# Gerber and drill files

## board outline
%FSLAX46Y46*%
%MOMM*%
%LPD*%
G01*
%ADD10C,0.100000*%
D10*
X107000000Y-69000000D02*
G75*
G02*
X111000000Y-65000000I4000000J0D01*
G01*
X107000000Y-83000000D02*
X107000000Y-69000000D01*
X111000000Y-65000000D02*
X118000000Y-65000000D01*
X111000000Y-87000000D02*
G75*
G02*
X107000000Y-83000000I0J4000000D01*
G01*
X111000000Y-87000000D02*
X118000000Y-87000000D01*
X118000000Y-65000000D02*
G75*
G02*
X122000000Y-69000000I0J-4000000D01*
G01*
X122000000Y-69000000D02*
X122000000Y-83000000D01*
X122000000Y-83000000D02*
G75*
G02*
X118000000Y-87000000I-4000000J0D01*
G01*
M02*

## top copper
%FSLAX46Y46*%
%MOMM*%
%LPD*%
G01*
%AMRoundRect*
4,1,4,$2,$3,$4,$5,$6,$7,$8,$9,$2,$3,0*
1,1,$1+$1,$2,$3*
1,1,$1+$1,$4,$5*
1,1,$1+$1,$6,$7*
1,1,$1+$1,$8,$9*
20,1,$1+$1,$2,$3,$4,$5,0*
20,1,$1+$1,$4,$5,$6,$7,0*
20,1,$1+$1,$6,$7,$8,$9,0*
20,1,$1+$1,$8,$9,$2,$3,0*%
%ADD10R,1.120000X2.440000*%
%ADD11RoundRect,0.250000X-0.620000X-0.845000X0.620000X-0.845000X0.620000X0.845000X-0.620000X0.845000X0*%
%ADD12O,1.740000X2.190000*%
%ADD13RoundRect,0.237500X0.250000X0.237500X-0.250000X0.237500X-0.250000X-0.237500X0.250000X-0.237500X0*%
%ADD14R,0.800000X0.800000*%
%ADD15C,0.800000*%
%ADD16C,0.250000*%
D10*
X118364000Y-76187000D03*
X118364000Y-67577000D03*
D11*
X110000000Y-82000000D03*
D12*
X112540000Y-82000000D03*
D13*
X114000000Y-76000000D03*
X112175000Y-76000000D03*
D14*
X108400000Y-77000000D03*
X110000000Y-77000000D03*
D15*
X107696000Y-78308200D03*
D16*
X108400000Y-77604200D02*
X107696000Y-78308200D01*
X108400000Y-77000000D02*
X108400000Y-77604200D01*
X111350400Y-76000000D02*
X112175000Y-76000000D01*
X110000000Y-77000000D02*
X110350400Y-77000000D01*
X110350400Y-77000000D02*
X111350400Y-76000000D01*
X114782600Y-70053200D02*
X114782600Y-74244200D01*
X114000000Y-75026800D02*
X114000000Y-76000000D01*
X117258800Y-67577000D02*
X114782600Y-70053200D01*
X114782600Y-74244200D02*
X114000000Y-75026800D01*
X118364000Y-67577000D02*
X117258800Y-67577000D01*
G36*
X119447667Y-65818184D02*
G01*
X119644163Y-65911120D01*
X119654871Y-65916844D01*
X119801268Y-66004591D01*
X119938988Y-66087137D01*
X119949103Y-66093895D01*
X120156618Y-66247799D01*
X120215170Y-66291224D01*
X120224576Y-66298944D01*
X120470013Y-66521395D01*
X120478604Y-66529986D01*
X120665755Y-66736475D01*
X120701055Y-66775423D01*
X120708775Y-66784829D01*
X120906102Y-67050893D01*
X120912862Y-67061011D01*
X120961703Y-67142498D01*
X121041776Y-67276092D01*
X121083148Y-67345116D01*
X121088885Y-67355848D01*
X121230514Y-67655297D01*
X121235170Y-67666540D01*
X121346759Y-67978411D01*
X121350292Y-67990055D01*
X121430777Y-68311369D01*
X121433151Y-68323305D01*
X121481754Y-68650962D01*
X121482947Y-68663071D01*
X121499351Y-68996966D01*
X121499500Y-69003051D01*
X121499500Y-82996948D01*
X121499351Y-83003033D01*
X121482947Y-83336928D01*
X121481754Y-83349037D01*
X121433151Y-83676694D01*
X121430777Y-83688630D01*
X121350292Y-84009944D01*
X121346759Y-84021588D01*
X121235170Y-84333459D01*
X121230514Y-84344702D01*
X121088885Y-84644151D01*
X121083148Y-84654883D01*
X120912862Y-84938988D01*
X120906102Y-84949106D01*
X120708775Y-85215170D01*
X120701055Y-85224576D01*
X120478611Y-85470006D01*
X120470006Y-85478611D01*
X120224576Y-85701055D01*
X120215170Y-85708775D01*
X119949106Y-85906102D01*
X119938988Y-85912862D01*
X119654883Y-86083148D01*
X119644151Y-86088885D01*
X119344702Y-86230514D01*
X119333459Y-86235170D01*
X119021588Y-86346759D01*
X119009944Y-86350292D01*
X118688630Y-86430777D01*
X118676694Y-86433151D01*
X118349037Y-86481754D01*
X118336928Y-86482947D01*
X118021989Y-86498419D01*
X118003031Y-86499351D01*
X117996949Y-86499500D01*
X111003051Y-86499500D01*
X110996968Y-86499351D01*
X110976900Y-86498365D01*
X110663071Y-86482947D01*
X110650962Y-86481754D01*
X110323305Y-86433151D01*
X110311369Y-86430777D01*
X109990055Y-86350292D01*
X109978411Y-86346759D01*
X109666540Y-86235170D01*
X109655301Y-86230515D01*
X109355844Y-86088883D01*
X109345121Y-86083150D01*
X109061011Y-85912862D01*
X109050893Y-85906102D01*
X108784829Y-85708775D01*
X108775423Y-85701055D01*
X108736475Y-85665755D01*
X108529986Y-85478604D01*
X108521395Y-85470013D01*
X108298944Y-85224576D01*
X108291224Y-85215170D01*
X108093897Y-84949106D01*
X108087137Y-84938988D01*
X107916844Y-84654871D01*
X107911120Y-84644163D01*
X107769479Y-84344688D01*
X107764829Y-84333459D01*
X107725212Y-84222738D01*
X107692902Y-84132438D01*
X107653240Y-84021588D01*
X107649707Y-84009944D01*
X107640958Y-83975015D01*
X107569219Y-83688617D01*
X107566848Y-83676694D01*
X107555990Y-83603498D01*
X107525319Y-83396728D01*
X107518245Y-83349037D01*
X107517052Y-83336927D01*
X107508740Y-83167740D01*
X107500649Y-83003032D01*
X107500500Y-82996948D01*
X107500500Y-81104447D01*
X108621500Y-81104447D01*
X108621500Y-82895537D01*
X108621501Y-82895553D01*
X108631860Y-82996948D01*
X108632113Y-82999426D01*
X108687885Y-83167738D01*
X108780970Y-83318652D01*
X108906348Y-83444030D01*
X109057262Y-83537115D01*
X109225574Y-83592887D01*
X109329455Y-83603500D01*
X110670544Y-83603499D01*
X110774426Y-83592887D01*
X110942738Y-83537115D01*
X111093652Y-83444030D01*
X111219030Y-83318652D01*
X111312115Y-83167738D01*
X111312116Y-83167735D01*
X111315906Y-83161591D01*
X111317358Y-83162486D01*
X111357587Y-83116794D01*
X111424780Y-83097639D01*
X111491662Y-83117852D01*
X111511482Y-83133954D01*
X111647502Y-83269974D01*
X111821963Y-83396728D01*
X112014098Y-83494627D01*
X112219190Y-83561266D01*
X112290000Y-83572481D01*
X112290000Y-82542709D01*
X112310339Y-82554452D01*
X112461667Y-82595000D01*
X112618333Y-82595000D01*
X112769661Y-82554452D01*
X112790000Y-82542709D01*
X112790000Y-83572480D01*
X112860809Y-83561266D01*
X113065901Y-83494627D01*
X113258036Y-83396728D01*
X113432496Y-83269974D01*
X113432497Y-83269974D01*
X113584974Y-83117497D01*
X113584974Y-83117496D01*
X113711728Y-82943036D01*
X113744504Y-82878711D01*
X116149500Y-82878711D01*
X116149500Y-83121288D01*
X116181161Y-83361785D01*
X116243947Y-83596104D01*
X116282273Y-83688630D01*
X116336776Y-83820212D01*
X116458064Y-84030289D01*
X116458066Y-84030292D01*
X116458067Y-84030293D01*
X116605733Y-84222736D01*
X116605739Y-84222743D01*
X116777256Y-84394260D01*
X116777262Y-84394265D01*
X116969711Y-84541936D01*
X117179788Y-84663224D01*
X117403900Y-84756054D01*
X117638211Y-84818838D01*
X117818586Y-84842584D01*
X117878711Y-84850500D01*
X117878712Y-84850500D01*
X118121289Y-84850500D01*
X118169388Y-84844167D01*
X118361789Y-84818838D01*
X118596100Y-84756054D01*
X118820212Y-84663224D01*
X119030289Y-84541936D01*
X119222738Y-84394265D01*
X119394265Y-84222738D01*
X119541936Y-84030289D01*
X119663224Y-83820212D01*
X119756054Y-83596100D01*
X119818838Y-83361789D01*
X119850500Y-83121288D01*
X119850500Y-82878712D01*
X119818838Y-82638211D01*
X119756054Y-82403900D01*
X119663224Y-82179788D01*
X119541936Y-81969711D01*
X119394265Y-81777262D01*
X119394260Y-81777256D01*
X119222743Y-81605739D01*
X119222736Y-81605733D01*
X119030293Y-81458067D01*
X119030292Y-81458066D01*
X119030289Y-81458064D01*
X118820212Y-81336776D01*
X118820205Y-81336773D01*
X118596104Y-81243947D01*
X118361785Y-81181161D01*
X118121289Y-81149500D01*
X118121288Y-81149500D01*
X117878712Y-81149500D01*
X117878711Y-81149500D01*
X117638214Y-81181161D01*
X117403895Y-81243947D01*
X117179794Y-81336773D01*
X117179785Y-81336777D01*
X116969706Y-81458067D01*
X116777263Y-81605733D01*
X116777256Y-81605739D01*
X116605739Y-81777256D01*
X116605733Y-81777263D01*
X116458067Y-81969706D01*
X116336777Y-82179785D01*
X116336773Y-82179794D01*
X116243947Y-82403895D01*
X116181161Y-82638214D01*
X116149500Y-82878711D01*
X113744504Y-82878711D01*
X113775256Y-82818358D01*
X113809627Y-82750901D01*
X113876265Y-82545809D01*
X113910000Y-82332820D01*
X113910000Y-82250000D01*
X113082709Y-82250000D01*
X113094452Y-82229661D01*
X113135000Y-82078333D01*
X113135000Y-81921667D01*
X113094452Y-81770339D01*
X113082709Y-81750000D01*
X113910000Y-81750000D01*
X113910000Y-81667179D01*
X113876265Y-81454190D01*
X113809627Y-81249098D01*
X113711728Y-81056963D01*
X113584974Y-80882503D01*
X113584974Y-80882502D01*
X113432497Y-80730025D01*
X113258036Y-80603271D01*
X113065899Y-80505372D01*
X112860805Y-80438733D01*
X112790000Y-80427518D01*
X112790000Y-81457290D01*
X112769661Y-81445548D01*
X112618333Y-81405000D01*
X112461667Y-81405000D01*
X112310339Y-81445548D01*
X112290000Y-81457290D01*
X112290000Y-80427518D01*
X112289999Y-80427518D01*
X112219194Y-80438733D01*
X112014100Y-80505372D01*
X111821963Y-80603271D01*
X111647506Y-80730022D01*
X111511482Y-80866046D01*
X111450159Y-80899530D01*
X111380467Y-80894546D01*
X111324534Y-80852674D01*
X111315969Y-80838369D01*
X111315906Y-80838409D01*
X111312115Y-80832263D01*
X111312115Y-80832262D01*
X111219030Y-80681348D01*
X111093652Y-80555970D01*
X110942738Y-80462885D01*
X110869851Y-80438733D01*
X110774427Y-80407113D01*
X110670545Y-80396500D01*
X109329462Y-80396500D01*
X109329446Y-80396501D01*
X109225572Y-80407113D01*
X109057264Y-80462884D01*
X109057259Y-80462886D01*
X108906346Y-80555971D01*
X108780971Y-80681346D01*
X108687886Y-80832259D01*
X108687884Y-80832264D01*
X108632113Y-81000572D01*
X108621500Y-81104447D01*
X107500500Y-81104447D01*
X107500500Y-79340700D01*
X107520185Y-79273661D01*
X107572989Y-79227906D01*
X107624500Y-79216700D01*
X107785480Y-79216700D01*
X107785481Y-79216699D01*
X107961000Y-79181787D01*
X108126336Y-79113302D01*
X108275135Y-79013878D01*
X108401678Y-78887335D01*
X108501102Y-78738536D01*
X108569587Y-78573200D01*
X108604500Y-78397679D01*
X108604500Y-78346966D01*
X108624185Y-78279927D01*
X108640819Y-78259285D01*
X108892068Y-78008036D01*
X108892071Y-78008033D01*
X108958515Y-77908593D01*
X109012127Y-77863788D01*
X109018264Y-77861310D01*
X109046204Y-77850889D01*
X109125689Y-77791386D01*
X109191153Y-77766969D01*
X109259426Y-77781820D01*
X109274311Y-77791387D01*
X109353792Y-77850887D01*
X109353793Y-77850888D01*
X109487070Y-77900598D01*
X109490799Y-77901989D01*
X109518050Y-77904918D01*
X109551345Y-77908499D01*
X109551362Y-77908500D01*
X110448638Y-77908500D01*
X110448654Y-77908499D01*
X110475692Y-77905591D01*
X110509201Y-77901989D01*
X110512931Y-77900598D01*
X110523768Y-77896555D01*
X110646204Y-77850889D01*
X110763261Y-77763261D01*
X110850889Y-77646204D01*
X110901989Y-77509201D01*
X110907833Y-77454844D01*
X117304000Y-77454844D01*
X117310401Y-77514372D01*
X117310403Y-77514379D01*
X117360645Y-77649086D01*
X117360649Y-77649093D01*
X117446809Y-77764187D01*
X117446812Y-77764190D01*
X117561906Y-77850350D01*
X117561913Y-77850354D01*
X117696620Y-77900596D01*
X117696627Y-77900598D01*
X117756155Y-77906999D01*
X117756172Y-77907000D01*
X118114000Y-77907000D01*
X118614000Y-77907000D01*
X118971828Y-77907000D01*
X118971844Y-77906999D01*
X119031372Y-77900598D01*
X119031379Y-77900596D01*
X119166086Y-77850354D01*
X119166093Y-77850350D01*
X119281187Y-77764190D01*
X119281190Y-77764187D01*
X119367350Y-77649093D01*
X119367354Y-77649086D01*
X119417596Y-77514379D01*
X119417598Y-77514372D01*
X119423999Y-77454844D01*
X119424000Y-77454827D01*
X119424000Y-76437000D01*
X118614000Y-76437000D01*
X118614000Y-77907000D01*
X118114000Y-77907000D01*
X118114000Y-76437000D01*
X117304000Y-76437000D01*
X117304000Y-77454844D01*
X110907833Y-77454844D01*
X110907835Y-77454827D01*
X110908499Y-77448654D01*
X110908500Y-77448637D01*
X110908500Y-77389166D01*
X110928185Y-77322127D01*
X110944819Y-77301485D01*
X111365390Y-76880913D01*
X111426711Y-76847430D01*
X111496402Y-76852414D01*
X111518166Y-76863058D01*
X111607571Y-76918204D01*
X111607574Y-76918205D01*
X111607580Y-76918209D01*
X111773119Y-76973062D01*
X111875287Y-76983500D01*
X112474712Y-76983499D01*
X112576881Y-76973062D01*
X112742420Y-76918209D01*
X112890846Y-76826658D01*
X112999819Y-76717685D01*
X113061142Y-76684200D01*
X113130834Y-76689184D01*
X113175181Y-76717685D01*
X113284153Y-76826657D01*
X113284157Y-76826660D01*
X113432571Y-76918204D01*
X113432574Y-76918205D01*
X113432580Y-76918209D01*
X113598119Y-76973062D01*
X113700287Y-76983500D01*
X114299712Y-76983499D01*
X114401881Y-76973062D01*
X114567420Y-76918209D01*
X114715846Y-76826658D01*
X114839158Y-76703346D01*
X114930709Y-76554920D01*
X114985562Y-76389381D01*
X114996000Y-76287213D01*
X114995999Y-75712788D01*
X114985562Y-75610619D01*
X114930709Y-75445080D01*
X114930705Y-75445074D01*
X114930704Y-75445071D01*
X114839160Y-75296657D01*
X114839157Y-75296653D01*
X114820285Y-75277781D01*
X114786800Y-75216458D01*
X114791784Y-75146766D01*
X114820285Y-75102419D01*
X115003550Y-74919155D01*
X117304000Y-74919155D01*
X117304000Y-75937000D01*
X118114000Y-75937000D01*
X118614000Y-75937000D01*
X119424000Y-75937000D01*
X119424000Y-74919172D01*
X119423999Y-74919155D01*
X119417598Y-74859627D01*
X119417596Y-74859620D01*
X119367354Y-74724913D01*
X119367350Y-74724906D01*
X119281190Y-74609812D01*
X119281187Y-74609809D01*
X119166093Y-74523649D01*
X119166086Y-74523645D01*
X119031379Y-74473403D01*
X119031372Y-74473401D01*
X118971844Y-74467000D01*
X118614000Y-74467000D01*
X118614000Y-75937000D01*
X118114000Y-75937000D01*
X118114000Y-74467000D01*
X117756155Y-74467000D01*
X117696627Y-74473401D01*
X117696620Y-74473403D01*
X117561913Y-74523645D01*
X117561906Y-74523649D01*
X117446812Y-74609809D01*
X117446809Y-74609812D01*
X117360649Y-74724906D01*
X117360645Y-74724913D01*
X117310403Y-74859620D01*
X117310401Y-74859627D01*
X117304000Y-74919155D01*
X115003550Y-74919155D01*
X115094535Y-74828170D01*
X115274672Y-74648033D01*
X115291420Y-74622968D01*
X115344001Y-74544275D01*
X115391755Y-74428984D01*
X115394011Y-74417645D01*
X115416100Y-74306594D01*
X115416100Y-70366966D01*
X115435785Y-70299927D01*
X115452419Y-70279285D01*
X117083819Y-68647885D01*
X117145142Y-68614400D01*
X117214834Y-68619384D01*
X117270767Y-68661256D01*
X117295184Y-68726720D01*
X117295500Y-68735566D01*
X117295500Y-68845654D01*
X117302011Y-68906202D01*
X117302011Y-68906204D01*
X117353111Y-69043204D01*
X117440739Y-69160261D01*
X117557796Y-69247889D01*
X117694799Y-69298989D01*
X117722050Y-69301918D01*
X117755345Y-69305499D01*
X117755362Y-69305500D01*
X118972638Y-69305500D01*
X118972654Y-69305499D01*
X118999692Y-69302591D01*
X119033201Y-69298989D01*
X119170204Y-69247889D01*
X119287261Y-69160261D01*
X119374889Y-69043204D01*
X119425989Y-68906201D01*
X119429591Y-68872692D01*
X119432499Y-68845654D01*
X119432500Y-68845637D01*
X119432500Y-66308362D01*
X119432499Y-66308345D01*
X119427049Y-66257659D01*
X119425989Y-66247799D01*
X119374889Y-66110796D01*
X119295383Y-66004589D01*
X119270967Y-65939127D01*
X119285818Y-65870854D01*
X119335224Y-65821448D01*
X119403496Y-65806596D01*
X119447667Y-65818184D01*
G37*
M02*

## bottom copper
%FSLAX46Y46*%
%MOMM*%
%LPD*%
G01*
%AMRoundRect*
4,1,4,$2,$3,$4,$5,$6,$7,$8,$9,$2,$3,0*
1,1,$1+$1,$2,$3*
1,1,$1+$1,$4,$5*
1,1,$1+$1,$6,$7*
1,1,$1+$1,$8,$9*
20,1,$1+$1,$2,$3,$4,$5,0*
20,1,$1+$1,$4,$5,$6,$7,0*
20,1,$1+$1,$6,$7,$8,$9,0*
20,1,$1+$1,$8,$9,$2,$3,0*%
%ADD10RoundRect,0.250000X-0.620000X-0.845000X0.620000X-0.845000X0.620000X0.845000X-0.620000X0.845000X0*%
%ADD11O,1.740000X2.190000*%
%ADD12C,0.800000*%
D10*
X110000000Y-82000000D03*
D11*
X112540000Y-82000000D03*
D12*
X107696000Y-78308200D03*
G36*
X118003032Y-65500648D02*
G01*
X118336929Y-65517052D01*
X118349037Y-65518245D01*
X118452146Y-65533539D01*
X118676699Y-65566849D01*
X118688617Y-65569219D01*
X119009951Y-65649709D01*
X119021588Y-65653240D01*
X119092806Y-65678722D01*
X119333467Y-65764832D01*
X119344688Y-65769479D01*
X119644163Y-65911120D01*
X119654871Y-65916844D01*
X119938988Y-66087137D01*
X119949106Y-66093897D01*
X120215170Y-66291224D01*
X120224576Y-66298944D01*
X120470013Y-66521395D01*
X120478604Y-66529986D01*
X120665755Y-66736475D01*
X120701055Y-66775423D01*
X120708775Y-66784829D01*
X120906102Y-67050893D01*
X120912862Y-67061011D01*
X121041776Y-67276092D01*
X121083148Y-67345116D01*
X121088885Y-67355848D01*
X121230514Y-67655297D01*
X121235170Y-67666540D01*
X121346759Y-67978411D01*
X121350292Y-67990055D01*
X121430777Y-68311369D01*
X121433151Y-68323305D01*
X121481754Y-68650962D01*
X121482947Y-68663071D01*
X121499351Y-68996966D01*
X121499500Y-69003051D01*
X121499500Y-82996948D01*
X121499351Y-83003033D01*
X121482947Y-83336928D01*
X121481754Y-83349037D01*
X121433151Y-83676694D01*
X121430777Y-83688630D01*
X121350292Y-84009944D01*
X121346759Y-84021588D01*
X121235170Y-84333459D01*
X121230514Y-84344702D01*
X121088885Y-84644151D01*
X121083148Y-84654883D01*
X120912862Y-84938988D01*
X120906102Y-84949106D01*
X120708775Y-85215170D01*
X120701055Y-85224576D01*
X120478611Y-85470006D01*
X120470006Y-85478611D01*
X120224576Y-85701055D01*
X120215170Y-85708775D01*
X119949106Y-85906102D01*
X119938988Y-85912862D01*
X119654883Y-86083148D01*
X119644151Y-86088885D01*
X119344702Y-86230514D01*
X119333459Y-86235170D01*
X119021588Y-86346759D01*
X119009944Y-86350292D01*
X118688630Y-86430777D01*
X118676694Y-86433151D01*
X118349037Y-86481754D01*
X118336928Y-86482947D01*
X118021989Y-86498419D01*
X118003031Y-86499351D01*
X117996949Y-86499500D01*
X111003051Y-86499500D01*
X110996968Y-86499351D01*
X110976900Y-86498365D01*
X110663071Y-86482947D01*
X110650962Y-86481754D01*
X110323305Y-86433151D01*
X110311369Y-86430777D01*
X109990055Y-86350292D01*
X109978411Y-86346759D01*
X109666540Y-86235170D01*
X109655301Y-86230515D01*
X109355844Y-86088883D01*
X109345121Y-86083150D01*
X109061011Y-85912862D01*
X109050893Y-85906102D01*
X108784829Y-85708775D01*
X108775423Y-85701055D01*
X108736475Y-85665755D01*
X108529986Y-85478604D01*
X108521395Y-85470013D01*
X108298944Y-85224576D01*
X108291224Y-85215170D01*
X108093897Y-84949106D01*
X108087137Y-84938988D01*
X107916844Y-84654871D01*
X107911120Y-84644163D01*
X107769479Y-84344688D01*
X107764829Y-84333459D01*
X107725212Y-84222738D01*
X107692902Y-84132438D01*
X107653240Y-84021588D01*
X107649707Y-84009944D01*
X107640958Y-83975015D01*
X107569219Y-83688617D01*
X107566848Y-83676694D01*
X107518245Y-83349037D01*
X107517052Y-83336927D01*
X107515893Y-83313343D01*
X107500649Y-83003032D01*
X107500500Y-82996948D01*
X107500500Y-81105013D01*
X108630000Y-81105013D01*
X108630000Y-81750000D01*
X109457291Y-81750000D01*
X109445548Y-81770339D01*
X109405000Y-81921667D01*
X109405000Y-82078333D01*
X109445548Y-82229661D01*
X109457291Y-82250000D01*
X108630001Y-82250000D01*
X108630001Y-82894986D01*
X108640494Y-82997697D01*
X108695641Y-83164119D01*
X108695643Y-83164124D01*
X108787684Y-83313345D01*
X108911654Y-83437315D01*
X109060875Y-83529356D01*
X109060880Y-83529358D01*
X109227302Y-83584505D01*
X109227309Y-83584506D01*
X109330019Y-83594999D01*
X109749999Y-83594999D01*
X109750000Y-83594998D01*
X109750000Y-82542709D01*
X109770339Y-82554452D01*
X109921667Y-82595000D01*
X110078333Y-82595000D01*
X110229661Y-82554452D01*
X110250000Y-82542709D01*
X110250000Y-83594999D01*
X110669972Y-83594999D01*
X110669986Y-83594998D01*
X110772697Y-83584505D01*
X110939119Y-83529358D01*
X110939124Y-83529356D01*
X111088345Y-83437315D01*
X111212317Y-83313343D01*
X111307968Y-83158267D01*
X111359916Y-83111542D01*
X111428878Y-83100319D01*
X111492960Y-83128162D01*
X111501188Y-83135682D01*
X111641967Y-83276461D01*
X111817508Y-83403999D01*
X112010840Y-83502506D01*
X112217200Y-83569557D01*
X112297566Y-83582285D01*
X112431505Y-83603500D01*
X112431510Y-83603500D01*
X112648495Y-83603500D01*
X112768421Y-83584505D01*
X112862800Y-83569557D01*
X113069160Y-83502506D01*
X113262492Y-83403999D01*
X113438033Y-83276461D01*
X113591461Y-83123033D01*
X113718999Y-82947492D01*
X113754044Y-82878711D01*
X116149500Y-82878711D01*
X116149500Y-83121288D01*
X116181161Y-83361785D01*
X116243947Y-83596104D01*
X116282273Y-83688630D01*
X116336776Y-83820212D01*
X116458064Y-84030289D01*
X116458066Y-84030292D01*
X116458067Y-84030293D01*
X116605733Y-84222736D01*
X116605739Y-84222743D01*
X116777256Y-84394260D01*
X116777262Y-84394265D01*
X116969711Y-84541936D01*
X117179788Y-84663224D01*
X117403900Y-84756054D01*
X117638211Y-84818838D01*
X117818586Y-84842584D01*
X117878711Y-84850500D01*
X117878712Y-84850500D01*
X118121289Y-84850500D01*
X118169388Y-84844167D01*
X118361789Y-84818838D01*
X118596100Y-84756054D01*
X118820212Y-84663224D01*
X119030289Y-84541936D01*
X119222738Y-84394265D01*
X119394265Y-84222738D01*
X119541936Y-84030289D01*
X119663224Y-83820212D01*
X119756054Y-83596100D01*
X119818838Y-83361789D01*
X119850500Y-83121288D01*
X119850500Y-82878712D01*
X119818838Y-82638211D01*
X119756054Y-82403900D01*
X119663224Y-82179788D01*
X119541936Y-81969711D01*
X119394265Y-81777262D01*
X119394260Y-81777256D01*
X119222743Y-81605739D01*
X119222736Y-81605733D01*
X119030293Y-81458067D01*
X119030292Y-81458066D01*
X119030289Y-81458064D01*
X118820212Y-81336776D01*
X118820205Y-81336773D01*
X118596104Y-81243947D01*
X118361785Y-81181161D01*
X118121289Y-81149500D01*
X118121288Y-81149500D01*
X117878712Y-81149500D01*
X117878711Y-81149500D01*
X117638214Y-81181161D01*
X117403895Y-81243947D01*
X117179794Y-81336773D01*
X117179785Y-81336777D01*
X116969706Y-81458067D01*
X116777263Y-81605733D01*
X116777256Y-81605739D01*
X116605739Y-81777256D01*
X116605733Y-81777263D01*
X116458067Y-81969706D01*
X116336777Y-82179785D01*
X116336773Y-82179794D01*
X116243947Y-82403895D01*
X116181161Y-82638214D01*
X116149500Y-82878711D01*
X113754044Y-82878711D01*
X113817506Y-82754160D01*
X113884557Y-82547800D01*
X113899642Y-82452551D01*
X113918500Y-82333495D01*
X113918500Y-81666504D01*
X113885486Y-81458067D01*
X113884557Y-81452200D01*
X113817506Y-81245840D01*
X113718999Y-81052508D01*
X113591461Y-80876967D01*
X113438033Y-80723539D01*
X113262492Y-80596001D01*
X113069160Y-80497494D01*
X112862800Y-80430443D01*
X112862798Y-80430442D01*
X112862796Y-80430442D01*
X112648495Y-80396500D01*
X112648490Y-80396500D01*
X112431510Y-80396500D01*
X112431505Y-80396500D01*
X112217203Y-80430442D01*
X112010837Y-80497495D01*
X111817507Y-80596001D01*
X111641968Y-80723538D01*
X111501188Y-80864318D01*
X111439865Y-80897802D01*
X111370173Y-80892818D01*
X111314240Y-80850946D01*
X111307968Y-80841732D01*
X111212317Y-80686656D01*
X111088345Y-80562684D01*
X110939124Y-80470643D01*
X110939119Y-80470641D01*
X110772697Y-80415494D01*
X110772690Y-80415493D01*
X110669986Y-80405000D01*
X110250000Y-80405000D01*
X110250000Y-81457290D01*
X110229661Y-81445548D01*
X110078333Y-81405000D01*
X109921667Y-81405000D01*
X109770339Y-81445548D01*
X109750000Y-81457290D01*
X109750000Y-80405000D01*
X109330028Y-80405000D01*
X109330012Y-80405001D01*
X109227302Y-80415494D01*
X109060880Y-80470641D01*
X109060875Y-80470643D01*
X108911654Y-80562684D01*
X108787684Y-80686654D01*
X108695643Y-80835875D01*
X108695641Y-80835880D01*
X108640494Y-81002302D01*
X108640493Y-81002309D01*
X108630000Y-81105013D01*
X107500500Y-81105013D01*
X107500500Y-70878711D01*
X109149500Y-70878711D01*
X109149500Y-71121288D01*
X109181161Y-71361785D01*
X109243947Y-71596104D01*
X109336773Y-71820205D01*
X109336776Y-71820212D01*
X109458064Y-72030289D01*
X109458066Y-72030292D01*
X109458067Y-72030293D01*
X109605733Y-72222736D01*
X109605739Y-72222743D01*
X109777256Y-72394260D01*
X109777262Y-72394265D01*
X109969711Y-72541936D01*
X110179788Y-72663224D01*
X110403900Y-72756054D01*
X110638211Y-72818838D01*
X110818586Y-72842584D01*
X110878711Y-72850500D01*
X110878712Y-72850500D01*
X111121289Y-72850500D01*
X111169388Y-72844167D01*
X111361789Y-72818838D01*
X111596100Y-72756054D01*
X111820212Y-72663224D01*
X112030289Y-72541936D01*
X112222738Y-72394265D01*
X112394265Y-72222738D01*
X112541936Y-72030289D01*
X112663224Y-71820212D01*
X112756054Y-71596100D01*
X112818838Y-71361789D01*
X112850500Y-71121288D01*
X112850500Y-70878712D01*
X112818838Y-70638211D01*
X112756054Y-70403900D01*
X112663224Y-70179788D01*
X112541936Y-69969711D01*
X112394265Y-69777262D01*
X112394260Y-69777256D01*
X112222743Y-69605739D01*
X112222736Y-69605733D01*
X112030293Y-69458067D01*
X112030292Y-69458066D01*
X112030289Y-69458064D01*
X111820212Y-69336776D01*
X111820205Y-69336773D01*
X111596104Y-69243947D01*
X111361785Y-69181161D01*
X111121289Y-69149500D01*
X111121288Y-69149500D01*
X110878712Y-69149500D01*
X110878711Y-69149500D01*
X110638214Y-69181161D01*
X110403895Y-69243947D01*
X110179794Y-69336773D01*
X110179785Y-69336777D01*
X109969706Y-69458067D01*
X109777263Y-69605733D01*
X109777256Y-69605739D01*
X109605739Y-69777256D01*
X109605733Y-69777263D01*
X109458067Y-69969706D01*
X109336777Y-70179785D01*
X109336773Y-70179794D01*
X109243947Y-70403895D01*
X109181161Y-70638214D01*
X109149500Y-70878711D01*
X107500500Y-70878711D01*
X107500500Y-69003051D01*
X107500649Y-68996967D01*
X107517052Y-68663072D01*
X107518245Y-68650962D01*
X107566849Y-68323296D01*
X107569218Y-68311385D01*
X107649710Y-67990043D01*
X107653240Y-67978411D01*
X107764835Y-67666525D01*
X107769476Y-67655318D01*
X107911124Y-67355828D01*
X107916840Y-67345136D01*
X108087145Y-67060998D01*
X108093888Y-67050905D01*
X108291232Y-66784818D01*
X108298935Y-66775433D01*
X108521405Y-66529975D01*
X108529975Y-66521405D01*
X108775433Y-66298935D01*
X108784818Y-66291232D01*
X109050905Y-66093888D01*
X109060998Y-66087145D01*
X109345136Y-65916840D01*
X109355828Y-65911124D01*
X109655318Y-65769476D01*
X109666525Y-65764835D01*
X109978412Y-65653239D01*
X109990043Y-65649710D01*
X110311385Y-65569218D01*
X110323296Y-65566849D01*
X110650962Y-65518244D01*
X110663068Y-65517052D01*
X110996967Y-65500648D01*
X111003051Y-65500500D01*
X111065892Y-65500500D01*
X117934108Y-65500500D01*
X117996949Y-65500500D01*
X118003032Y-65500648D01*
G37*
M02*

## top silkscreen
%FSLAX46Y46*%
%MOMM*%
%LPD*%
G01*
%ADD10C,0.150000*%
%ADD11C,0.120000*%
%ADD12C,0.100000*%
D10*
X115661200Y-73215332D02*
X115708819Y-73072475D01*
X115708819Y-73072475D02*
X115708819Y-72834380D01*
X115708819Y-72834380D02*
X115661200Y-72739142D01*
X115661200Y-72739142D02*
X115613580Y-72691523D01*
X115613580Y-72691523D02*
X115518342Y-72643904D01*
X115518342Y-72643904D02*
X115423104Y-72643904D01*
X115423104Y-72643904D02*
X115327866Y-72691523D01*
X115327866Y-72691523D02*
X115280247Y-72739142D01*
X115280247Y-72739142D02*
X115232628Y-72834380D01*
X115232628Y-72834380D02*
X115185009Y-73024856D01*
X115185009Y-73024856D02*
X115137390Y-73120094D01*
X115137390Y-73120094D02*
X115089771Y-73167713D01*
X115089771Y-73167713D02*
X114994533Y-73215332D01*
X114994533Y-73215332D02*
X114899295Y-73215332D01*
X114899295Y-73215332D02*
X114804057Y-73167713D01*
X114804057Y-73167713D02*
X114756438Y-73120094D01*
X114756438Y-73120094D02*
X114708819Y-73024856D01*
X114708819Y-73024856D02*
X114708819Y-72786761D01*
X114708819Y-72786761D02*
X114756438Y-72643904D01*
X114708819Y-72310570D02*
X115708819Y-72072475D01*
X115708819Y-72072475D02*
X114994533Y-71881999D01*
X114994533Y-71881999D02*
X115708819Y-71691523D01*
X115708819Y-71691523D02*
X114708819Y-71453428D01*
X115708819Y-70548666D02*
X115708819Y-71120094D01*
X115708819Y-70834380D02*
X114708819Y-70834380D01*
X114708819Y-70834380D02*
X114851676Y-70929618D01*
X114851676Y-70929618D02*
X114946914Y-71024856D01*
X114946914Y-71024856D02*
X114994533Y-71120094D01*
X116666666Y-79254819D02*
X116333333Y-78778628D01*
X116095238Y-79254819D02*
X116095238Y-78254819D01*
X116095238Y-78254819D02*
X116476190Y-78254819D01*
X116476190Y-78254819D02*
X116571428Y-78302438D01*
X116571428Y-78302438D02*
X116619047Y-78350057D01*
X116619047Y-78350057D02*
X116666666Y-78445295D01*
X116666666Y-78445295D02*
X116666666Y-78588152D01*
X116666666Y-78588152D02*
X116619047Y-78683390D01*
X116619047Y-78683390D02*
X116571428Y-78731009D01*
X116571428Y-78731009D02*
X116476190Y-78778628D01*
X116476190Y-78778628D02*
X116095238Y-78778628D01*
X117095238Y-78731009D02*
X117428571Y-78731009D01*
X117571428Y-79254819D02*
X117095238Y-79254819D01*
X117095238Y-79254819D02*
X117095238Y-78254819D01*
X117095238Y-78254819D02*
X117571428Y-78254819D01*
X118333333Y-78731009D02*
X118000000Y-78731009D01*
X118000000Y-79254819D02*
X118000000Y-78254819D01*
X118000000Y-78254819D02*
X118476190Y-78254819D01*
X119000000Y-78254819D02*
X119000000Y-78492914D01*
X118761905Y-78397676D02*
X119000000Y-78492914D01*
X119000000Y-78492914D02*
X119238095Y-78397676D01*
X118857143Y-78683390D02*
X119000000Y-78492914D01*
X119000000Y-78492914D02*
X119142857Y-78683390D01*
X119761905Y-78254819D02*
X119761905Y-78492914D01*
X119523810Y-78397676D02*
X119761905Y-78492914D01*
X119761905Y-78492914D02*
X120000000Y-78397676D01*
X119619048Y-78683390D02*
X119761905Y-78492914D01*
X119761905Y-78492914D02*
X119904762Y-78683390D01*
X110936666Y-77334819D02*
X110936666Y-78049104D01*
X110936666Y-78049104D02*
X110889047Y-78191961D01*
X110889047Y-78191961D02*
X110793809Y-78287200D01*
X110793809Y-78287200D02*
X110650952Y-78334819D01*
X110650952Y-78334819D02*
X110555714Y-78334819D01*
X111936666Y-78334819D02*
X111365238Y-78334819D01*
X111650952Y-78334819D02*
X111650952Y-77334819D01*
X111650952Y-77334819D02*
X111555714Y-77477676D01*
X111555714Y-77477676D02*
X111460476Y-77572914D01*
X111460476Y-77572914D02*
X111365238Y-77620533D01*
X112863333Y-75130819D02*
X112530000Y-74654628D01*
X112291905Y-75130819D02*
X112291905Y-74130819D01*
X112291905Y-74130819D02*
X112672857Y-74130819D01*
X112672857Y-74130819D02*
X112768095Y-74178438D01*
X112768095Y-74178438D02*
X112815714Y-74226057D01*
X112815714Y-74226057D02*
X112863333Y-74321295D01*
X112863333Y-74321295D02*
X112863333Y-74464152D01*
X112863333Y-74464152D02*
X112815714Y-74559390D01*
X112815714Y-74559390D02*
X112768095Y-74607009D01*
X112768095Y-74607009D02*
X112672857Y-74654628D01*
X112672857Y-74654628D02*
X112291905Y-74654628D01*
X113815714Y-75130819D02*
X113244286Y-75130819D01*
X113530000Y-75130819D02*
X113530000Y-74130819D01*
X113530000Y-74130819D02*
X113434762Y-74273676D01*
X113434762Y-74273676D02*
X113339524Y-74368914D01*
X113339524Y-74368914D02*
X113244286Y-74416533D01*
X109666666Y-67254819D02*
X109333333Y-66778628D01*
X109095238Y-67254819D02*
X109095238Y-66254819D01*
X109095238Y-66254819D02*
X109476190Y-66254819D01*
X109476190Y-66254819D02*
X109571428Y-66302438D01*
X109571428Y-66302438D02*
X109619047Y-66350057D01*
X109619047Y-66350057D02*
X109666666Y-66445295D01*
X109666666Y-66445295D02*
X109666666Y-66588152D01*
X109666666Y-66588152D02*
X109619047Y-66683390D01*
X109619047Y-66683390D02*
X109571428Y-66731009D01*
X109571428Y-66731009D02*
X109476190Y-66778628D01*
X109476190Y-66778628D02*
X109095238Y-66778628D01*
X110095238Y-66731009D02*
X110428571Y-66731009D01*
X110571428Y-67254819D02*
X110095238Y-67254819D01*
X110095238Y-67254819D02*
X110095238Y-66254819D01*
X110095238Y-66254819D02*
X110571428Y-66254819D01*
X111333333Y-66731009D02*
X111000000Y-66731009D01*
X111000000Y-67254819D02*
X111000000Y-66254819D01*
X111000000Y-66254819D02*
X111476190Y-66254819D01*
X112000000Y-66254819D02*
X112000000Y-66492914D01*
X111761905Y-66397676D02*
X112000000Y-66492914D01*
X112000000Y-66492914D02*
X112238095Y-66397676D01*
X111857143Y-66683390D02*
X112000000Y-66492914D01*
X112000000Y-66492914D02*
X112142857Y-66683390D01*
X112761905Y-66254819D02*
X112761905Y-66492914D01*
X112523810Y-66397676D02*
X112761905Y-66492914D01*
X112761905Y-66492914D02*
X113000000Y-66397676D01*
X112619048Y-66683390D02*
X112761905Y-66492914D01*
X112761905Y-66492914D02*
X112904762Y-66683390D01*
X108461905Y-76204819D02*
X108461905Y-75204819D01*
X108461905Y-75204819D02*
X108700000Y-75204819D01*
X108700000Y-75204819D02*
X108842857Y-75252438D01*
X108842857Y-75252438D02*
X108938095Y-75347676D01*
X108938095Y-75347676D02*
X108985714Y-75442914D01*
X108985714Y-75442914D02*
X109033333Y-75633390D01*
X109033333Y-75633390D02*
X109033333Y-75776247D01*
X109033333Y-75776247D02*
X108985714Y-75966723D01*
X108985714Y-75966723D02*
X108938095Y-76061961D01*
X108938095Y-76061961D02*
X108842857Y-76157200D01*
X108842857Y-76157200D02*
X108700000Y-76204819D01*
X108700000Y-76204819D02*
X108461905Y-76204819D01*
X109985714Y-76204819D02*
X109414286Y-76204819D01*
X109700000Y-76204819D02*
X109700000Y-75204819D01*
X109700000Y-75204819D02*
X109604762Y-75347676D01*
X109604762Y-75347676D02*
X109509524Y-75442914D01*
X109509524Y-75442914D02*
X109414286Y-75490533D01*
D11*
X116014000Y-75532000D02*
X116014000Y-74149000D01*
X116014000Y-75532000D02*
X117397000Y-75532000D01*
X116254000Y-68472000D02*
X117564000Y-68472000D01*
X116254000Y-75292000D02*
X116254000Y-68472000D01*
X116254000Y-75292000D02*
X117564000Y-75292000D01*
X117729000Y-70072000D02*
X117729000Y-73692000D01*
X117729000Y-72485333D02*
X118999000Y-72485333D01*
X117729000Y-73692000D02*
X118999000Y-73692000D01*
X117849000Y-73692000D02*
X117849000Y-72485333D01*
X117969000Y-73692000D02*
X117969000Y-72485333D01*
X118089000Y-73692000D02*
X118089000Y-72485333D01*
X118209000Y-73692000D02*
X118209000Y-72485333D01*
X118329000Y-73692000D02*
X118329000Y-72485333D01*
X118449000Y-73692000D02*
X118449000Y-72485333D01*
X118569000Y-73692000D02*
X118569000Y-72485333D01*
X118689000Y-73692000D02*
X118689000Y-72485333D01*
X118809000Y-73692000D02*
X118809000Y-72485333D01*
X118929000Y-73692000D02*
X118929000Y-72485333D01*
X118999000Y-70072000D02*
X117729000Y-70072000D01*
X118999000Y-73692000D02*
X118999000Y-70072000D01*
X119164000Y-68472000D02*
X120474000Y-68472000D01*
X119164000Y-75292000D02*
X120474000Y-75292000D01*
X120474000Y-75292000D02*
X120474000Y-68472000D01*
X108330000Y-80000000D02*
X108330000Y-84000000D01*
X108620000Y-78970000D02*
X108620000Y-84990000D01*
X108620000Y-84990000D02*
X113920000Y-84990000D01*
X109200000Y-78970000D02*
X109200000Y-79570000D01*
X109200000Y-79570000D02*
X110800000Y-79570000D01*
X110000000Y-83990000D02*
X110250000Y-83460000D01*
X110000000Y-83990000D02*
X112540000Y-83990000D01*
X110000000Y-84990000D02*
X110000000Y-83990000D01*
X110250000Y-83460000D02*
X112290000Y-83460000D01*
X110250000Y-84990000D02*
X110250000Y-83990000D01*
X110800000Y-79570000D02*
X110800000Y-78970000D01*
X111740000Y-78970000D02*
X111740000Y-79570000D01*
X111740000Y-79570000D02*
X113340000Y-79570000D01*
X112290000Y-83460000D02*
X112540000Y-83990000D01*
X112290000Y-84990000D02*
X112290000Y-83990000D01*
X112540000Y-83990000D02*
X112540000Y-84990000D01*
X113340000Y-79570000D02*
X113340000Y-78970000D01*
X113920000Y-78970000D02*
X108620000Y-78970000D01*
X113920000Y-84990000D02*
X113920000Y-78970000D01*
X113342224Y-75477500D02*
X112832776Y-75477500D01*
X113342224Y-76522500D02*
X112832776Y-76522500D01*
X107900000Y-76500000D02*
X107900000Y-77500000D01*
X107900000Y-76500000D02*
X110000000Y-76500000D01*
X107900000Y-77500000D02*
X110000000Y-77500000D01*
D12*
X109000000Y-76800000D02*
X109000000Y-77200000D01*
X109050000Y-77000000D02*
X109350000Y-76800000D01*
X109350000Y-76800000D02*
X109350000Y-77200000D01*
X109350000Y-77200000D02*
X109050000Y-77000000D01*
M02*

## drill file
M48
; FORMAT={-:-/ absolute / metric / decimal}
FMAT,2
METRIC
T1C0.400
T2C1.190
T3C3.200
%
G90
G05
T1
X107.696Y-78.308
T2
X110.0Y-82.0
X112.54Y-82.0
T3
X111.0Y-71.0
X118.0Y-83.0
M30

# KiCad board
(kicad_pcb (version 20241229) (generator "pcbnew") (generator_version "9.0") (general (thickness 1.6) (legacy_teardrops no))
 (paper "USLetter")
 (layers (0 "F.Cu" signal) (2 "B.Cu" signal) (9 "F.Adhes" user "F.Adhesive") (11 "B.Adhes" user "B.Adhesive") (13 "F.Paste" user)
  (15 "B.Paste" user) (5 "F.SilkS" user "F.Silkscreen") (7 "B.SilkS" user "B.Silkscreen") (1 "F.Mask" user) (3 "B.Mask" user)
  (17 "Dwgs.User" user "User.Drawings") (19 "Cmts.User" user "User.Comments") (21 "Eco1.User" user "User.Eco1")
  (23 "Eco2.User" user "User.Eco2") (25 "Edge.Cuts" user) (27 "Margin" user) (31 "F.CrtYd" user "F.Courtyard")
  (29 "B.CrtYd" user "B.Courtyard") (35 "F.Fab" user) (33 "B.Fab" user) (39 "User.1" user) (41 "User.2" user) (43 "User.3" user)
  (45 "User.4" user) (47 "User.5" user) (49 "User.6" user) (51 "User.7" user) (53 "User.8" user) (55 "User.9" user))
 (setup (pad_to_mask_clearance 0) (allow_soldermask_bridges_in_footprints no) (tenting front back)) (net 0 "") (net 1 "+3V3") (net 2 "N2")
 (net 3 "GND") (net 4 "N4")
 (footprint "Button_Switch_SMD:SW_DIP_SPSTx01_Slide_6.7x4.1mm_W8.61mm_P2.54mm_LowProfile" (layer "F.Cu") (at 118.364 71.882 90)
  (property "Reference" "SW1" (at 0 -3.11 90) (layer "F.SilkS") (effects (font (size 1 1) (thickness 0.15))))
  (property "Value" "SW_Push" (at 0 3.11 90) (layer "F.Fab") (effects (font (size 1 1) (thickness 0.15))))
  (fp_line (start -3.65 -2.35) (end -2.267 -2.35) (stroke (width 0.12) (type solid)) (layer "F.SilkS"))
  (fp_line (start -3.65 -2.35) (end -3.65 -0.967) (stroke (width 0.12) (type solid)) (layer "F.SilkS"))
  (fp_line (start 3.41 -2.11) (end 3.41 -0.8) (stroke (width 0.12) (type solid)) (layer "F.SilkS"))
  (fp_line (start -3.41 -2.11) (end 3.41 -2.11) (stroke (width 0.12) (type solid)) (layer "F.SilkS"))
  (fp_line (start -3.41 -2.11) (end -3.41 -0.8) (stroke (width 0.12) (type solid)) (layer "F.SilkS"))
  (fp_line (start 1.81 -0.635) (end -1.81 -0.635) (stroke (width 0.12) (type solid)) (layer "F.SilkS"))
  (fp_line (start -0.603333 -0.635) (end -0.603333 0.635) (stroke (width 0.12) (type solid)) (layer "F.SilkS"))
  (fp_line (start -1.81 -0.635) (end -1.81 0.635) (stroke (width 0.12) (type solid)) (layer "F.SilkS"))
  (fp_line (start -1.81 -0.515) (end -0.603333 -0.515) (stroke (width 0.12) (type solid)) (layer "F.SilkS"))
  (fp_line (start -1.81 -0.395) (end -0.603333 -0.395) (stroke (width 0.12) (type solid)) (layer "F.SilkS"))
  (fp_line (start -1.81 -0.275) (end -0.603333 -0.275) (stroke (width 0.12) (type solid)) (layer "F.SilkS"))
  (fp_line (start -1.81 -0.155) (end -0.603333 -0.155) (stroke (width 0.12) (type solid)) (layer "F.SilkS"))
  (fp_line (start -1.81 -0.035) (end -0.603333 -0.035) (stroke (width 0.12) (type solid)) (layer "F.SilkS"))
  (fp_line (start -1.81 0.085) (end -0.603333 0.085) (stroke (width 0.12) (type solid)) (layer "F.SilkS"))
  (fp_line (start -1.81 0.205) (end -0.603333 0.205) (stroke (width 0.12) (type solid)) (layer "F.SilkS"))
  (fp_line (start -1.81 0.325) (end -0.603333 0.325) (stroke (width 0.12) (type solid)) (layer "F.SilkS"))
  (fp_line (start -1.81 0.445) (end -0.603333 0.445) (stroke (width 0.12) (type solid)) (layer "F.SilkS"))
  (fp_line (start -1.81 0.565) (end -0.603333 0.565) (stroke (width 0.12) (type solid)) (layer "F.SilkS"))
  (fp_line (start 1.81 0.635) (end 1.81 -0.635) (stroke (width 0.12) (type solid)) (layer "F.SilkS"))
  (fp_line (start -1.81 0.635) (end 1.81 0.635) (stroke (width 0.12) (type solid)) (layer "F.SilkS"))
  (fp_line (start 3.41 0.8) (end 3.41 2.11) (stroke (width 0.12) (type solid)) (layer "F.SilkS"))
  (fp_line (start -3.41 0.8) (end -3.41 2.11) (stroke (width 0.12) (type solid)) (layer "F.SilkS"))
  (fp_line (start -3.41 2.11) (end 3.41 2.11) (stroke (width 0.12) (type solid)) (layer "F.SilkS"))
  (pad "1" smd rect (at -4.305 0 90) (size 2.44 1.12) (layers "F.Cu" "F.Mask" "F.Paste") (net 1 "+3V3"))
  (pad "2" smd rect (at 4.305 0 90) (size 2.44 1.12) (layers "F.Cu" "F.Mask" "F.Paste") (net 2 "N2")))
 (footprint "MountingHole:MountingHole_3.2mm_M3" (layer "F.Cu") (at 118 83)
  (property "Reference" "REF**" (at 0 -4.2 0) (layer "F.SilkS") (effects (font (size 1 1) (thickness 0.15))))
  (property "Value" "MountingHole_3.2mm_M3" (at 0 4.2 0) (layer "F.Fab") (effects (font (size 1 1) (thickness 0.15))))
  (pad "" np_thru_hole circle (at 0 0) (size 3.2 3.2) (drill 3.2) (layers "*.Cu" "*.Mask")))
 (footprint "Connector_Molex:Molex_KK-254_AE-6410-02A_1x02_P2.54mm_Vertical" (layer "F.Cu") (at 110 82)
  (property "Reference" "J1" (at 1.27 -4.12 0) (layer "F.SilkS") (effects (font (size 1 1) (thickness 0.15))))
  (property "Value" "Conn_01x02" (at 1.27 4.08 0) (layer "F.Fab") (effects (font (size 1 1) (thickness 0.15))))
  (fp_line (start -1.67 -2) (end -1.67 2) (stroke (width 0.12) (type solid)) (layer "F.SilkS"))
  (fp_line (start -1.38 -3.03) (end -1.38 2.99) (stroke (width 0.12) (type solid)) (layer "F.SilkS"))
  (fp_line (start -1.38 2.99) (end 3.92 2.99) (stroke (width 0.12) (type solid)) (layer "F.SilkS"))
  (fp_line (start -0.8 -3.03) (end -0.8 -2.43) (stroke (width 0.12) (type solid)) (layer "F.SilkS"))
  (fp_line (start -0.8 -2.43) (end 0.8 -2.43) (stroke (width 0.12) (type solid)) (layer "F.SilkS"))
  (fp_line (start 0 1.99) (end 0.25 1.46) (stroke (width 0.12) (type solid)) (layer "F.SilkS"))
  (fp_line (start 0 1.99) (end 2.54 1.99) (stroke (width 0.12) (type solid)) (layer "F.SilkS"))
  (fp_line (start 0 2.99) (end 0 1.99) (stroke (width 0.12) (type solid)) (layer "F.SilkS"))
  (fp_line (start 0.25 1.46) (end 2.29 1.46) (stroke (width 0.12) (type solid)) (layer "F.SilkS"))
  (fp_line (start 0.25 2.99) (end 0.25 1.99) (stroke (width 0.12) (type solid)) (layer "F.SilkS"))
  (fp_line (start 0.8 -2.43) (end 0.8 -3.03) (stroke (width 0.12) (type solid)) (layer "F.SilkS"))
  (fp_line (start 1.74 -3.03) (end 1.74 -2.43) (stroke (width 0.12) (type solid)) (layer "F.SilkS"))
  (fp_line (start 1.74 -2.43) (end 3.34 -2.43) (stroke (width 0.12) (type solid)) (layer "F.SilkS"))
  (fp_line (start 2.29 1.46) (end 2.54 1.99) (stroke (width 0.12) (type solid)) (layer "F.SilkS"))
  (fp_line (start 2.29 2.99) (end 2.29 1.99) (stroke (width 0.12) (type solid)) (layer "F.SilkS"))
  (fp_line (start 2.54 1.99) (end 2.54 2.99) (stroke (width 0.12) (type solid)) (layer "F.SilkS"))
  (fp_line (start 3.34 -2.43) (end 3.34 -3.03) (stroke (width 0.12) (type solid)) (layer "F.SilkS"))
  (fp_line (start 3.92 -3.03) (end -1.38 -3.03) (stroke (width 0.12) (type solid)) (layer "F.SilkS"))
  (fp_line (start 3.92 2.99) (end 3.92 -3.03) (stroke (width 0.12) (type solid)) (layer "F.SilkS"))
  (pad "1" thru_hole roundrect (at 0 0) (size 1.74 2.19) (drill 1.19) (layers "*.Cu" "*.Mask") (remove_unused_layers no)
   (roundrect_rratio 0.143678) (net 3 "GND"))
  (pad "2" thru_hole oval (at 2.54 0) (size 1.74 2.19) (drill 1.19) (layers "*.Cu" "*.Mask") (remove_unused_layers no) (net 1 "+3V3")))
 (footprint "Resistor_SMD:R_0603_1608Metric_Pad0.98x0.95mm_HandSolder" (layer "F.Cu") (at 113.0875 76 180)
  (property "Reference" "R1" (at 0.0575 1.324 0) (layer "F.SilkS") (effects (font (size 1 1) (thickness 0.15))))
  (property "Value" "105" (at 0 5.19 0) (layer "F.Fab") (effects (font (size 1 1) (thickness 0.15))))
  (fp_line (start -0.254724 0.5225) (end 0.254724 0.5225) (stroke (width 0.12) (type solid)) (layer "F.SilkS"))
  (fp_line (start -0.254724 -0.5225) (end 0.254724 -0.5225) (stroke (width 0.12) (type solid)) (layer "F.SilkS"))
  (pad "1" smd roundrect (at -0.9125 0 180) (size 0.975 0.95) (layers "F.Cu" "F.Mask" "F.Paste") (roundrect_rratio 0.25) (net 2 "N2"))
  (pad "2" smd roundrect (at 0.9125 0 180) (size 0.975 0.95) (layers "F.Cu" "F.Mask" "F.Paste") (roundrect_rratio 0.25) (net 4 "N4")))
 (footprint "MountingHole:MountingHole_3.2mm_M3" (layer "F.Cu") (at 111 71)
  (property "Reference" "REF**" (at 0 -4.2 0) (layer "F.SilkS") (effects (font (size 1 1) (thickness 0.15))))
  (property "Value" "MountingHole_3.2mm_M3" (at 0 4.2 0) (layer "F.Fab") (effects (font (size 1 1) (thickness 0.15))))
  (pad "" np_thru_hole circle (at 0 0) (size 3.2 3.2) (drill 3.2) (layers "*.Cu" "*.Mask")))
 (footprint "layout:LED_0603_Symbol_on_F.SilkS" (layer "F.Cu") (at 109.2 77)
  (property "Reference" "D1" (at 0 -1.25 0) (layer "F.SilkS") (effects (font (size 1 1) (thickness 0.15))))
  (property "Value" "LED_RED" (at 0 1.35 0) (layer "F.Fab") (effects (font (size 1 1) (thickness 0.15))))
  (fp_line (start -1.3 -0.5) (end -1.3 0.5) (stroke (width 0.12) (type solid)) (layer "F.SilkS"))
  (fp_line (start -1.3 -0.5) (end 0.8 -0.5) (stroke (width 0.12) (type solid)) (layer "F.SilkS"))
  (fp_line (start -1.3 0.5) (end 0.8 0.5) (stroke (width 0.12) (type solid)) (layer "F.SilkS"))
  (fp_line (start -0.2 -0.2) (end -0.2 0.2) (stroke (width 0.1) (type solid)) (layer "F.SilkS"))
  (fp_line (start -0.15 0) (end 0.15 -0.2) (stroke (width 0.1) (type solid)) (layer "F.SilkS"))
  (fp_line (start 0.15 -0.2) (end 0.15 0.2) (stroke (width 0.1) (type solid)) (layer "F.SilkS"))
  (fp_line (start 0.15 0.2) (end -0.15 0) (stroke (width 0.1) (type solid)) (layer "F.SilkS"))
  (pad "1" smd rect (at -0.8 0 180) (size 0.8 0.8) (layers "F.Cu" "F.Mask" "F.Paste") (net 3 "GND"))
  (pad "2" smd rect (at 0.8 0 180) (size 0.8 0.8) (layers "F.Cu" "F.Mask" "F.Paste") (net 4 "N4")))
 (gr_arc (start 107 69) (mid 108.171573 66.171573) (end 111 65) (stroke (width 0.1) (type default)) (layer "Edge.Cuts"))
 (gr_line (start 107 83) (end 107 69) (stroke (width 0.1) (type default)) (layer "Edge.Cuts"))
 (gr_line (start 111 65) (end 118 65) (stroke (width 0.1) (type default)) (layer "Edge.Cuts"))
 (gr_arc (start 111 87) (mid 108.171573 85.828427) (end 107 83) (stroke (width 0.1) (type default)) (layer "Edge.Cuts"))
 (gr_line (start 111 87) (end 118 87) (stroke (width 0.1) (type default)) (layer "Edge.Cuts"))
 (gr_arc (start 118 65) (mid 120.828427 66.171573) (end 122 69) (stroke (width 0.1) (type default)) (layer "Edge.Cuts"))
 (gr_line (start 122 69) (end 122 83) (stroke (width 0.1) (type default)) (layer "Edge.Cuts"))
 (gr_arc (start 122 83) (mid 120.828427 85.828427) (end 118 87) (stroke (width 0.1) (type default)) (layer "Edge.Cuts"))
 (segment (start 108.4 77.6042) (end 107.696 78.3082) (width 0.25) (layer "F.Cu") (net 3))
 (segment (start 108.4 77) (end 108.4 77.6042) (width 0.25) (layer "F.Cu") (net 3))
 (via (at 107.696 78.3082) (size 0.8) (drill 0.4) (layers "F.Cu" "B.Cu") (free yes) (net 3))
 (segment (start 111.3504 76) (end 112.175 76) (width 0.25) (layer "F.Cu") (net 4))
 (segment (start 110 77) (end 110.3504 77) (width 0.25) (layer "F.Cu") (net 4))
 (segment (start 110.3504 77) (end 111.3504 76) (width 0.25) (layer "F.Cu") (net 4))
 (segment (start 114.7826 70.0532) (end 114.7826 74.2442) (width 0.25) (layer "F.Cu") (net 2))
 (segment (start 114 75.0268) (end 114 76) (width 0.25) (layer "F.Cu") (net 2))
 (segment (start 117.2588 67.577) (end 114.7826 70.0532) (width 0.25) (layer "F.Cu") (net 2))
 (segment (start 114.7826 74.2442) (end 114 75.0268) (width 0.25) (layer "F.Cu") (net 2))
 (segment (start 118.364 67.577) (end 117.2588 67.577) (width 0.25) (layer "F.Cu") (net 2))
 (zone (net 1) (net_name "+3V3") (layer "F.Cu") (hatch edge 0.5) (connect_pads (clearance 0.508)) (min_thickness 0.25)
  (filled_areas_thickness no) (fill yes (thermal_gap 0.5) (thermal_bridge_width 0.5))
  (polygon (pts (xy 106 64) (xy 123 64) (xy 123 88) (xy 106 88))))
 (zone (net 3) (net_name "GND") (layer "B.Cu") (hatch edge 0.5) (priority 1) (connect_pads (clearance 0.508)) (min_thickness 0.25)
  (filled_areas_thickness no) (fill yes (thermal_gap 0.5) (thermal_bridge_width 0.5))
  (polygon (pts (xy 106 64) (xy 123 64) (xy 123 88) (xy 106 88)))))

